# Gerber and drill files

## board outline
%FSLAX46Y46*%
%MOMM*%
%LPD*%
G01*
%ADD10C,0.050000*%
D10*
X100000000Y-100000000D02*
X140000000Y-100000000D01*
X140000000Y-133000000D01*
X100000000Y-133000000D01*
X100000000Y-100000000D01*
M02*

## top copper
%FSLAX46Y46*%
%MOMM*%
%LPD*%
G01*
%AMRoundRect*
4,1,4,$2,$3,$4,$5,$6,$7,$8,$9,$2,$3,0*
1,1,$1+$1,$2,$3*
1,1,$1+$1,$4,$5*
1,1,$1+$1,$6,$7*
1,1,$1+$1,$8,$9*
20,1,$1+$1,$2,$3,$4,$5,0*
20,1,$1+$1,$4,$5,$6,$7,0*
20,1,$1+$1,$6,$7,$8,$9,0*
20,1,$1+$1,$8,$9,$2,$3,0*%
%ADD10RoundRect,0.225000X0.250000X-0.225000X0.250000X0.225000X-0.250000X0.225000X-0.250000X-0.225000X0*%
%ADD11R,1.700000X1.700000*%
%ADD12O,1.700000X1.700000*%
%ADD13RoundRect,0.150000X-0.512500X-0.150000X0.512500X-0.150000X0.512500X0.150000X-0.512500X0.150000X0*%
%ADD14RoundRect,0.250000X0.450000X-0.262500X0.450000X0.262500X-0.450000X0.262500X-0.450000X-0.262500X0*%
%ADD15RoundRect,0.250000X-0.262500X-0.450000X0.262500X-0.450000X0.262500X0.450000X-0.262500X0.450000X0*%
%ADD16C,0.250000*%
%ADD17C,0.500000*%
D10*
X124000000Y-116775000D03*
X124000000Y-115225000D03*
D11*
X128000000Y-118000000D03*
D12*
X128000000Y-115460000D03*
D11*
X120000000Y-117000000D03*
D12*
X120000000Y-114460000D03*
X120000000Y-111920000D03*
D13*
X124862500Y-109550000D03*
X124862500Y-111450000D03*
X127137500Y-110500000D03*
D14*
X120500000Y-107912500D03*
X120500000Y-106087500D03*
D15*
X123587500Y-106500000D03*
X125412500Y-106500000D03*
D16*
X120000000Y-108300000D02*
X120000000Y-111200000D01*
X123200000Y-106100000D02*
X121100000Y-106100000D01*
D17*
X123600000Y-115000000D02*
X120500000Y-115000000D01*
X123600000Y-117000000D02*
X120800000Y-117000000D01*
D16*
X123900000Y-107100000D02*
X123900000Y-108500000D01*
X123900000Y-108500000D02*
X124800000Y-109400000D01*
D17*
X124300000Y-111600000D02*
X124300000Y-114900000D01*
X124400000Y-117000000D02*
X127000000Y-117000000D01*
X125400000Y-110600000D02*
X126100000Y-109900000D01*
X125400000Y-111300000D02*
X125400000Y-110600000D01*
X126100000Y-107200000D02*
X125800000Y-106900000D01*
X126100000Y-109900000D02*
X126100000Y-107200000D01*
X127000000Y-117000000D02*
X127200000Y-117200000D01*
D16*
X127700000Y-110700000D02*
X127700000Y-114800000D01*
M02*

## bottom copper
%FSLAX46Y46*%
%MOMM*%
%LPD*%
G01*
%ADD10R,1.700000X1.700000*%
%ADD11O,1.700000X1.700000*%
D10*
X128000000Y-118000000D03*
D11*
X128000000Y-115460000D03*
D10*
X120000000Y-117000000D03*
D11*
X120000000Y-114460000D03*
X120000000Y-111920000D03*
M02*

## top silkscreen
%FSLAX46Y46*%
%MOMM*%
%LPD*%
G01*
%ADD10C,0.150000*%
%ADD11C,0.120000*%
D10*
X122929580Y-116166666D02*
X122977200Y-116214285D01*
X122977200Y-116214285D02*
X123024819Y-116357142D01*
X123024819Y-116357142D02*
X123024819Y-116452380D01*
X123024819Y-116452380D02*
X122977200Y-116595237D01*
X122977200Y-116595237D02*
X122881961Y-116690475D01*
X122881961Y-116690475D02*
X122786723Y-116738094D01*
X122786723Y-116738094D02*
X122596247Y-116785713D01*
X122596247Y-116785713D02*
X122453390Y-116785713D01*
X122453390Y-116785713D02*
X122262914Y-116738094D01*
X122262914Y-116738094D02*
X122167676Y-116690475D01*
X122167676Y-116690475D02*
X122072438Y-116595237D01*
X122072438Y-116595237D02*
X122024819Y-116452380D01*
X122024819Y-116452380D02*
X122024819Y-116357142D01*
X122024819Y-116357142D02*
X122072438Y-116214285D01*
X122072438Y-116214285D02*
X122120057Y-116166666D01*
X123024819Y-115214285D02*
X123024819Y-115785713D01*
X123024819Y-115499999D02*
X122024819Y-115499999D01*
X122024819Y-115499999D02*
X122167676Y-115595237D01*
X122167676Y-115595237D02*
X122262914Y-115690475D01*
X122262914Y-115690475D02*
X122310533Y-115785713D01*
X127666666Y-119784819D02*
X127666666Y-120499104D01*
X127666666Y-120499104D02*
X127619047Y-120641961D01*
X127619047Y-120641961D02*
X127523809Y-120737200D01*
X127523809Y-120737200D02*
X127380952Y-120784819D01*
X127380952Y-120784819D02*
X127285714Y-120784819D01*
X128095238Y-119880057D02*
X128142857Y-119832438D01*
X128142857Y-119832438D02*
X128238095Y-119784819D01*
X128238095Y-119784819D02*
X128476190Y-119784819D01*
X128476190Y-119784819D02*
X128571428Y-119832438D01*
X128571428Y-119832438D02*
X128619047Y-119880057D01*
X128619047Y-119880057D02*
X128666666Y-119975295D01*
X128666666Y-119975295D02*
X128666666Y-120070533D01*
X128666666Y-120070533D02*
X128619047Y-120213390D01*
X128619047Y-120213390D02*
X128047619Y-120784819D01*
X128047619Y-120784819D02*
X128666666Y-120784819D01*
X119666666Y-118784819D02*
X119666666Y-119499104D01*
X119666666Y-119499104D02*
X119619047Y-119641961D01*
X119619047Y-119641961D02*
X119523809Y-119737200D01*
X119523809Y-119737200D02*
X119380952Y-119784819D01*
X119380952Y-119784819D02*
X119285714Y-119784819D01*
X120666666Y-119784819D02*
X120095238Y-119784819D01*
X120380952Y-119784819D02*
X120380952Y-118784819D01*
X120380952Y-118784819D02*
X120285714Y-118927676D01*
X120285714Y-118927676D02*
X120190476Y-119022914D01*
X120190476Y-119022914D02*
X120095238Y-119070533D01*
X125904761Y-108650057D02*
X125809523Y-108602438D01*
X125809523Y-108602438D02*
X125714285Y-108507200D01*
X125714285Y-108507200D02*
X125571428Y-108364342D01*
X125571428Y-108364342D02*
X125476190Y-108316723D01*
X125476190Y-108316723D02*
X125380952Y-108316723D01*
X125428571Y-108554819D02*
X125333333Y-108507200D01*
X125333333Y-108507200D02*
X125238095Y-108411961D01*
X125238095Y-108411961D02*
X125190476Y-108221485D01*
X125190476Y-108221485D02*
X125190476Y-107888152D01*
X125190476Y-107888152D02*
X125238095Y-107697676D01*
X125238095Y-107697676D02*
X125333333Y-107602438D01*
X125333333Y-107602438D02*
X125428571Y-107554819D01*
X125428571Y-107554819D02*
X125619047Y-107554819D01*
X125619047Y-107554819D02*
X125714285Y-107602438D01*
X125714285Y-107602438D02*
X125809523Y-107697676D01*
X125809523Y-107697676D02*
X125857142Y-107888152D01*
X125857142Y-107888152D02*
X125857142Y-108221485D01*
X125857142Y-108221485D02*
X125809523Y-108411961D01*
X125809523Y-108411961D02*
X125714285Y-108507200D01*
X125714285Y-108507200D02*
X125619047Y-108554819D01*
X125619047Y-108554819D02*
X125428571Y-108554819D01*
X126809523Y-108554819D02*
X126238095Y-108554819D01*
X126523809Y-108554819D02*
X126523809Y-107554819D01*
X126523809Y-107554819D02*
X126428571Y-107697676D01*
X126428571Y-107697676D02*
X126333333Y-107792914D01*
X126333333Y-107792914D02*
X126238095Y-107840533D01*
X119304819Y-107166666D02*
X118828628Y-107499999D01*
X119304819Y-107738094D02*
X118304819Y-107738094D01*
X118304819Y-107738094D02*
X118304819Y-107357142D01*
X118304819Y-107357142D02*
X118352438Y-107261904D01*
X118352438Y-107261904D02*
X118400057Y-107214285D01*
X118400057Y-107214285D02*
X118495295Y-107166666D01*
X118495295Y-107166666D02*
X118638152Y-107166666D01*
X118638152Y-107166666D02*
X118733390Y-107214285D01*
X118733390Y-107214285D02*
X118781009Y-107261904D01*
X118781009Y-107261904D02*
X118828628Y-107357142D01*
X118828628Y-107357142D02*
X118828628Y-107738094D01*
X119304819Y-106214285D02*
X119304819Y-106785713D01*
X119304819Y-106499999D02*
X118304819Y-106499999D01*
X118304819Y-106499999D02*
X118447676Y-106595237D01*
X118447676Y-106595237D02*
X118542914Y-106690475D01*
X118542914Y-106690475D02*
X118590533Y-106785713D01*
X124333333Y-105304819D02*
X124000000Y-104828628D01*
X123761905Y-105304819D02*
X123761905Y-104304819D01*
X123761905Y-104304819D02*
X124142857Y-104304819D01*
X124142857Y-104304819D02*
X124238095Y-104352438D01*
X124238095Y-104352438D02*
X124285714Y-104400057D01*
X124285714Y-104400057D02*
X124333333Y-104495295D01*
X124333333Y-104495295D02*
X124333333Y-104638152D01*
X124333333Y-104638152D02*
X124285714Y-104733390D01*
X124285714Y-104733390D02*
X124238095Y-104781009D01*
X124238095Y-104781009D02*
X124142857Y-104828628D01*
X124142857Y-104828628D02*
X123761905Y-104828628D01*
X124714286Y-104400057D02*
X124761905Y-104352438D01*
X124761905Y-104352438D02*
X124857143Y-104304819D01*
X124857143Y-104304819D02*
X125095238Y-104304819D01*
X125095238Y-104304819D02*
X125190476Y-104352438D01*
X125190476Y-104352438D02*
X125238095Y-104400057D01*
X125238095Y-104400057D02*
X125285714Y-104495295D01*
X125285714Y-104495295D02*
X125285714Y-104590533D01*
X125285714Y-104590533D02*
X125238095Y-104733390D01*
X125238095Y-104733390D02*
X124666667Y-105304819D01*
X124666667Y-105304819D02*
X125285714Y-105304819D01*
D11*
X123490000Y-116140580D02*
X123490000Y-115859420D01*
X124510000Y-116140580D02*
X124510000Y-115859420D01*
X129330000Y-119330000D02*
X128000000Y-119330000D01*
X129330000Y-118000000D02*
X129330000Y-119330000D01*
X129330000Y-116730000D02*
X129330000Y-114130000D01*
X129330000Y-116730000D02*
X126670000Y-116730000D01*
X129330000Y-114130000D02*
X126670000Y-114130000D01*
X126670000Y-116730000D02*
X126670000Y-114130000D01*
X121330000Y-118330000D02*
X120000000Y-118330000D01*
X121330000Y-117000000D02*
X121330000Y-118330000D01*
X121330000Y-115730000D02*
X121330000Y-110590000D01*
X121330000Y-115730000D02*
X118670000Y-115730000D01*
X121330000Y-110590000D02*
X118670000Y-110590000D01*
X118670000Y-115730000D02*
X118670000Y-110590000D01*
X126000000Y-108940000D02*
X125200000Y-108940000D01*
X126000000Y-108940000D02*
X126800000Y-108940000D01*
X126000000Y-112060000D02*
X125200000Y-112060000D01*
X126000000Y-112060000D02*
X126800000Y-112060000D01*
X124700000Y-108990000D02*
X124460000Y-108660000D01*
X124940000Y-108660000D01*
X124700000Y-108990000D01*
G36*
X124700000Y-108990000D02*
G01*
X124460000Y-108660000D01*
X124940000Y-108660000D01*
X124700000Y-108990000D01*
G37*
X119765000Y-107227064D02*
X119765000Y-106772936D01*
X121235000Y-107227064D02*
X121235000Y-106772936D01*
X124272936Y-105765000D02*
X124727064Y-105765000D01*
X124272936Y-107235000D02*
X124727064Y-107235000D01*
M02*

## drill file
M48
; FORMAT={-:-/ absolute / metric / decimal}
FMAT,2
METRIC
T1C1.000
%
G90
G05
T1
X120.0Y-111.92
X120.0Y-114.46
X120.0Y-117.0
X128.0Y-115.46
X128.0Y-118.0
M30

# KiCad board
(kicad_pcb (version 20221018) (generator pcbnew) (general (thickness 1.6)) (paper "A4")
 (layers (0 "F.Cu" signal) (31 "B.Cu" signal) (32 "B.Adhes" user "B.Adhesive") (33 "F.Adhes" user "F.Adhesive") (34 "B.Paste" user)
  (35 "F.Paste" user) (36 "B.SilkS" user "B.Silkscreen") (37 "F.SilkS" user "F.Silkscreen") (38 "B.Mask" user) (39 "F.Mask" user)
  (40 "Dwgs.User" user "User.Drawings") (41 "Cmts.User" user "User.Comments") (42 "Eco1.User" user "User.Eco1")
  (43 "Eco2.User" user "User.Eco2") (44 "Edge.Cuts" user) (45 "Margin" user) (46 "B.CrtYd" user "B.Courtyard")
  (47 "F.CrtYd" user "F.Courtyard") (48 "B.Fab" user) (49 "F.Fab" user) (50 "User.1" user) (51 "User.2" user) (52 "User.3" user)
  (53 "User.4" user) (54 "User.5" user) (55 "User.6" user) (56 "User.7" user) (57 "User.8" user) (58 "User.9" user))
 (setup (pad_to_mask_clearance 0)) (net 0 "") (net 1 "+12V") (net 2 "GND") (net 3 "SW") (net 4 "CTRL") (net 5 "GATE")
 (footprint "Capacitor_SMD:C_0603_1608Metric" (layer "F.Cu") (at 124 116 90)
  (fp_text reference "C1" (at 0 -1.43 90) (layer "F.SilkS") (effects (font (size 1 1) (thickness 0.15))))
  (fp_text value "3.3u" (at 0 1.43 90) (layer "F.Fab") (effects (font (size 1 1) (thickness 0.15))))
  (fp_line (start -0.14058 -0.51) (end 0.14058 -0.51) (stroke (width 0.12) (type solid)) (layer "F.SilkS"))
  (fp_line (start -0.14058 0.51) (end 0.14058 0.51) (stroke (width 0.12) (type solid)) (layer "F.SilkS"))
  (pad "1" smd roundrect (at -0.775 0 90) (size 0.9 0.95) (layers "F.Cu" "F.Paste" "F.Mask") (roundrect_rratio 0.25) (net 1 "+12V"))
  (pad "2" smd roundrect (at 0.775 0 90) (size 0.9 0.95) (layers "F.Cu" "F.Paste" "F.Mask") (roundrect_rratio 0.25) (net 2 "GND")))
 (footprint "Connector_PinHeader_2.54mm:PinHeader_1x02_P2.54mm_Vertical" (layer "F.Cu") (at 128 118 180)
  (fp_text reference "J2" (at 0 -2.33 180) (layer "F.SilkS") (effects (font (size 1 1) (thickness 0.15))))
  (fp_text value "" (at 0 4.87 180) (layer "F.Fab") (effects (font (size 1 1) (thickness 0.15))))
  (fp_line (start -1.33 -1.33) (end 0 -1.33) (stroke (width 0.12) (type solid)) (layer "F.SilkS"))
  (fp_line (start -1.33 0) (end -1.33 -1.33) (stroke (width 0.12) (type solid)) (layer "F.SilkS"))
  (fp_line (start -1.33 1.27) (end -1.33 3.87) (stroke (width 0.12) (type solid)) (layer "F.SilkS"))
  (fp_line (start -1.33 1.27) (end 1.33 1.27) (stroke (width 0.12) (type solid)) (layer "F.SilkS"))
  (fp_line (start -1.33 3.87) (end 1.33 3.87) (stroke (width 0.12) (type solid)) (layer "F.SilkS"))
  (fp_line (start 1.33 1.27) (end 1.33 3.87) (stroke (width 0.12) (type solid)) (layer "F.SilkS"))
  (pad "1" thru_hole rect (at 0 0 180) (size 1.7 1.7) (drill 1) (layers "*.Cu" "*.Mask") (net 1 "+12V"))
  (pad "2" thru_hole oval (at 0 2.54 180) (size 1.7 1.7) (drill 1) (layers "*.Cu" "*.Mask") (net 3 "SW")))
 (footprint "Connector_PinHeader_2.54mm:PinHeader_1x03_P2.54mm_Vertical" (layer "F.Cu") (at 120 117 180)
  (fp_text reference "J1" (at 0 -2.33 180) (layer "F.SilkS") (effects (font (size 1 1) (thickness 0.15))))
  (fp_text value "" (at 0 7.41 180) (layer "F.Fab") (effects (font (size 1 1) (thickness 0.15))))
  (fp_line (start -1.33 -1.33) (end 0 -1.33) (stroke (width 0.12) (type solid)) (layer "F.SilkS"))
  (fp_line (start -1.33 0) (end -1.33 -1.33) (stroke (width 0.12) (type solid)) (layer "F.SilkS"))
  (fp_line (start -1.33 1.27) (end -1.33 6.41) (stroke (width 0.12) (type solid)) (layer "F.SilkS"))
  (fp_line (start -1.33 1.27) (end 1.33 1.27) (stroke (width 0.12) (type solid)) (layer "F.SilkS"))
  (fp_line (start -1.33 6.41) (end 1.33 6.41) (stroke (width 0.12) (type solid)) (layer "F.SilkS"))
  (fp_line (start 1.33 1.27) (end 1.33 6.41) (stroke (width 0.12) (type solid)) (layer "F.SilkS"))
  (pad "1" thru_hole rect (at 0 0 180) (size 1.7 1.7) (drill 1) (layers "*.Cu" "*.Mask") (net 1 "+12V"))
  (pad "2" thru_hole oval (at 0 2.54 180) (size 1.7 1.7) (drill 1) (layers "*.Cu" "*.Mask") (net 2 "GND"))
  (pad "3" thru_hole oval (at 0 5.08 180) (size 1.7 1.7) (drill 1) (layers "*.Cu" "*.Mask") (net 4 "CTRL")))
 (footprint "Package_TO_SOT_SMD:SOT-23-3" (layer "F.Cu") (at 126 110.5)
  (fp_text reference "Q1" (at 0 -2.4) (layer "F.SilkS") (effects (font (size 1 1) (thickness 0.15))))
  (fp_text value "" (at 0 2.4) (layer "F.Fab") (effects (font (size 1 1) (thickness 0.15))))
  (fp_line (start 0 -1.56) (end -0.8 -1.56) (stroke (width 0.12) (type solid)) (layer "F.SilkS"))
  (fp_line (start 0 -1.56) (end 0.8 -1.56) (stroke (width 0.12) (type solid)) (layer "F.SilkS"))
  (fp_line (start 0 1.56) (end -0.8 1.56) (stroke (width 0.12) (type solid)) (layer "F.SilkS"))
  (fp_line (start 0 1.56) (end 0.8 1.56) (stroke (width 0.12) (type solid)) (layer "F.SilkS"))
  (fp_poly
   (pts (xy -1.3 -1.51) (xy -1.54 -1.84) (xy -1.06 -1.84) (xy -1.3 -1.51)) (stroke (width 0.12) (type solid)) (fill solid) (layer "F.SilkS"))
  (pad "1" smd roundrect (at -1.1375 -0.95) (size 1.325 0.6) (layers "F.Cu" "F.Paste" "F.Mask") (roundrect_rratio 0.25) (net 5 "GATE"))
  (pad "2" smd roundrect (at -1.1375 0.95) (size 1.325 0.6) (layers "F.Cu" "F.Paste" "F.Mask") (roundrect_rratio 0.25) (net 2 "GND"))
  (pad "3" smd roundrect (at 1.1375 0) (size 1.325 0.6) (layers "F.Cu" "F.Paste" "F.Mask") (roundrect_rratio 0.25) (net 3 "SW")))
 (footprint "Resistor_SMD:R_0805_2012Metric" (layer "F.Cu") (at 120.5 107 90)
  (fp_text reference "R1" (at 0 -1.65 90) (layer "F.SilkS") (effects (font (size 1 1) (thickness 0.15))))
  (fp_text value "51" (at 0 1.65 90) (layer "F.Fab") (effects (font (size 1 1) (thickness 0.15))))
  (fp_line (start -0.227064 -0.735) (end 0.227064 -0.735) (stroke (width 0.12) (type solid)) (layer "F.SilkS"))
  (fp_line (start -0.227064 0.735) (end 0.227064 0.735) (stroke (width 0.12) (type solid)) (layer "F.SilkS"))
  (pad "1" smd roundrect (at -0.9125 0 90) (size 1.025 1.4) (layers "F.Cu" "F.Paste" "F.Mask") (roundrect_rratio 0.243902) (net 4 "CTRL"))
  (pad "2" smd roundrect (at 0.9125 0 90) (size 1.025 1.4) (layers "F.Cu" "F.Paste" "F.Mask") (roundrect_rratio 0.243902) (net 5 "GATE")))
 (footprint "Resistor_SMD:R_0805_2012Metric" (layer "F.Cu") (at 124.5 106.5)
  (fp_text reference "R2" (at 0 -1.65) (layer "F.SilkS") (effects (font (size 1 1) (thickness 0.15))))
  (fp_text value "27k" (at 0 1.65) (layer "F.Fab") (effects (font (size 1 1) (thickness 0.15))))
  (fp_line (start -0.227064 -0.735) (end 0.227064 -0.735) (stroke (width 0.12) (type solid)) (layer "F.SilkS"))
  (fp_line (start -0.227064 0.735) (end 0.227064 0.735) (stroke (width 0.12) (type solid)) (layer "F.SilkS"))
  (pad "1" smd roundrect (at -0.9125 0) (size 1.025 1.4) (layers "F.Cu" "F.Paste" "F.Mask") (roundrect_rratio 0.243902) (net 5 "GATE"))
  (pad "2" smd roundrect (at 0.9125 0) (size 1.025 1.4) (layers "F.Cu" "F.Paste" "F.Mask") (roundrect_rratio 0.243902) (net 2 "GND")))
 (gr_rect (start 100 100) (end 140 133) (stroke (width 0.05) (type default)) (fill none) (layer "Edge.Cuts"))
 (segment (start 120 108.3) (end 120 111.2) (width 0.25) (layer "F.Cu") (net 4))
 (segment (start 123.2 106.1) (end 121.1 106.1) (width 0.25) (layer "F.Cu") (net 5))
 (segment (start 123.6 115) (end 120.5 115) (width 0.5) (layer "F.Cu") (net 2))
 (segment (start 123.6 117) (end 120.8 117) (width 0.5) (layer "F.Cu") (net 1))
 (segment (start 123.9 107.1) (end 123.9 108.5) (width 0.25) (layer "F.Cu") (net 5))
 (segment (start 123.9 108.5) (end 124.8 109.4) (width 0.25) (layer "F.Cu") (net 5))
 (segment (start 124.3 111.6) (end 124.3 114.9) (width 0.5) (layer "F.Cu") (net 2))
 (segment (start 124.4 117) (end 127 117) (width 0.5) (layer "F.Cu") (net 1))
 (segment (start 125.4 110.6) (end 126.1 109.9) (width 0.5) (layer "F.Cu") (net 2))
 (segment (start 125.4 111.3) (end 125.4 110.6) (width 0.5) (layer "F.Cu") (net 2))
 (segment (start 126.1 107.2) (end 125.8 106.9) (width 0.5) (layer "F.Cu") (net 2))
 (segment (start 126.1 109.9) (end 126.1 107.2) (width 0.5) (layer "F.Cu") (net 2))
 (segment (start 127 117) (end 127.2 117.2) (width 0.5) (layer "F.Cu") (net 1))
 (segment (start 127.7 110.7) (end 127.7 114.8) (width 0.25) (layer "F.Cu") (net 3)))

